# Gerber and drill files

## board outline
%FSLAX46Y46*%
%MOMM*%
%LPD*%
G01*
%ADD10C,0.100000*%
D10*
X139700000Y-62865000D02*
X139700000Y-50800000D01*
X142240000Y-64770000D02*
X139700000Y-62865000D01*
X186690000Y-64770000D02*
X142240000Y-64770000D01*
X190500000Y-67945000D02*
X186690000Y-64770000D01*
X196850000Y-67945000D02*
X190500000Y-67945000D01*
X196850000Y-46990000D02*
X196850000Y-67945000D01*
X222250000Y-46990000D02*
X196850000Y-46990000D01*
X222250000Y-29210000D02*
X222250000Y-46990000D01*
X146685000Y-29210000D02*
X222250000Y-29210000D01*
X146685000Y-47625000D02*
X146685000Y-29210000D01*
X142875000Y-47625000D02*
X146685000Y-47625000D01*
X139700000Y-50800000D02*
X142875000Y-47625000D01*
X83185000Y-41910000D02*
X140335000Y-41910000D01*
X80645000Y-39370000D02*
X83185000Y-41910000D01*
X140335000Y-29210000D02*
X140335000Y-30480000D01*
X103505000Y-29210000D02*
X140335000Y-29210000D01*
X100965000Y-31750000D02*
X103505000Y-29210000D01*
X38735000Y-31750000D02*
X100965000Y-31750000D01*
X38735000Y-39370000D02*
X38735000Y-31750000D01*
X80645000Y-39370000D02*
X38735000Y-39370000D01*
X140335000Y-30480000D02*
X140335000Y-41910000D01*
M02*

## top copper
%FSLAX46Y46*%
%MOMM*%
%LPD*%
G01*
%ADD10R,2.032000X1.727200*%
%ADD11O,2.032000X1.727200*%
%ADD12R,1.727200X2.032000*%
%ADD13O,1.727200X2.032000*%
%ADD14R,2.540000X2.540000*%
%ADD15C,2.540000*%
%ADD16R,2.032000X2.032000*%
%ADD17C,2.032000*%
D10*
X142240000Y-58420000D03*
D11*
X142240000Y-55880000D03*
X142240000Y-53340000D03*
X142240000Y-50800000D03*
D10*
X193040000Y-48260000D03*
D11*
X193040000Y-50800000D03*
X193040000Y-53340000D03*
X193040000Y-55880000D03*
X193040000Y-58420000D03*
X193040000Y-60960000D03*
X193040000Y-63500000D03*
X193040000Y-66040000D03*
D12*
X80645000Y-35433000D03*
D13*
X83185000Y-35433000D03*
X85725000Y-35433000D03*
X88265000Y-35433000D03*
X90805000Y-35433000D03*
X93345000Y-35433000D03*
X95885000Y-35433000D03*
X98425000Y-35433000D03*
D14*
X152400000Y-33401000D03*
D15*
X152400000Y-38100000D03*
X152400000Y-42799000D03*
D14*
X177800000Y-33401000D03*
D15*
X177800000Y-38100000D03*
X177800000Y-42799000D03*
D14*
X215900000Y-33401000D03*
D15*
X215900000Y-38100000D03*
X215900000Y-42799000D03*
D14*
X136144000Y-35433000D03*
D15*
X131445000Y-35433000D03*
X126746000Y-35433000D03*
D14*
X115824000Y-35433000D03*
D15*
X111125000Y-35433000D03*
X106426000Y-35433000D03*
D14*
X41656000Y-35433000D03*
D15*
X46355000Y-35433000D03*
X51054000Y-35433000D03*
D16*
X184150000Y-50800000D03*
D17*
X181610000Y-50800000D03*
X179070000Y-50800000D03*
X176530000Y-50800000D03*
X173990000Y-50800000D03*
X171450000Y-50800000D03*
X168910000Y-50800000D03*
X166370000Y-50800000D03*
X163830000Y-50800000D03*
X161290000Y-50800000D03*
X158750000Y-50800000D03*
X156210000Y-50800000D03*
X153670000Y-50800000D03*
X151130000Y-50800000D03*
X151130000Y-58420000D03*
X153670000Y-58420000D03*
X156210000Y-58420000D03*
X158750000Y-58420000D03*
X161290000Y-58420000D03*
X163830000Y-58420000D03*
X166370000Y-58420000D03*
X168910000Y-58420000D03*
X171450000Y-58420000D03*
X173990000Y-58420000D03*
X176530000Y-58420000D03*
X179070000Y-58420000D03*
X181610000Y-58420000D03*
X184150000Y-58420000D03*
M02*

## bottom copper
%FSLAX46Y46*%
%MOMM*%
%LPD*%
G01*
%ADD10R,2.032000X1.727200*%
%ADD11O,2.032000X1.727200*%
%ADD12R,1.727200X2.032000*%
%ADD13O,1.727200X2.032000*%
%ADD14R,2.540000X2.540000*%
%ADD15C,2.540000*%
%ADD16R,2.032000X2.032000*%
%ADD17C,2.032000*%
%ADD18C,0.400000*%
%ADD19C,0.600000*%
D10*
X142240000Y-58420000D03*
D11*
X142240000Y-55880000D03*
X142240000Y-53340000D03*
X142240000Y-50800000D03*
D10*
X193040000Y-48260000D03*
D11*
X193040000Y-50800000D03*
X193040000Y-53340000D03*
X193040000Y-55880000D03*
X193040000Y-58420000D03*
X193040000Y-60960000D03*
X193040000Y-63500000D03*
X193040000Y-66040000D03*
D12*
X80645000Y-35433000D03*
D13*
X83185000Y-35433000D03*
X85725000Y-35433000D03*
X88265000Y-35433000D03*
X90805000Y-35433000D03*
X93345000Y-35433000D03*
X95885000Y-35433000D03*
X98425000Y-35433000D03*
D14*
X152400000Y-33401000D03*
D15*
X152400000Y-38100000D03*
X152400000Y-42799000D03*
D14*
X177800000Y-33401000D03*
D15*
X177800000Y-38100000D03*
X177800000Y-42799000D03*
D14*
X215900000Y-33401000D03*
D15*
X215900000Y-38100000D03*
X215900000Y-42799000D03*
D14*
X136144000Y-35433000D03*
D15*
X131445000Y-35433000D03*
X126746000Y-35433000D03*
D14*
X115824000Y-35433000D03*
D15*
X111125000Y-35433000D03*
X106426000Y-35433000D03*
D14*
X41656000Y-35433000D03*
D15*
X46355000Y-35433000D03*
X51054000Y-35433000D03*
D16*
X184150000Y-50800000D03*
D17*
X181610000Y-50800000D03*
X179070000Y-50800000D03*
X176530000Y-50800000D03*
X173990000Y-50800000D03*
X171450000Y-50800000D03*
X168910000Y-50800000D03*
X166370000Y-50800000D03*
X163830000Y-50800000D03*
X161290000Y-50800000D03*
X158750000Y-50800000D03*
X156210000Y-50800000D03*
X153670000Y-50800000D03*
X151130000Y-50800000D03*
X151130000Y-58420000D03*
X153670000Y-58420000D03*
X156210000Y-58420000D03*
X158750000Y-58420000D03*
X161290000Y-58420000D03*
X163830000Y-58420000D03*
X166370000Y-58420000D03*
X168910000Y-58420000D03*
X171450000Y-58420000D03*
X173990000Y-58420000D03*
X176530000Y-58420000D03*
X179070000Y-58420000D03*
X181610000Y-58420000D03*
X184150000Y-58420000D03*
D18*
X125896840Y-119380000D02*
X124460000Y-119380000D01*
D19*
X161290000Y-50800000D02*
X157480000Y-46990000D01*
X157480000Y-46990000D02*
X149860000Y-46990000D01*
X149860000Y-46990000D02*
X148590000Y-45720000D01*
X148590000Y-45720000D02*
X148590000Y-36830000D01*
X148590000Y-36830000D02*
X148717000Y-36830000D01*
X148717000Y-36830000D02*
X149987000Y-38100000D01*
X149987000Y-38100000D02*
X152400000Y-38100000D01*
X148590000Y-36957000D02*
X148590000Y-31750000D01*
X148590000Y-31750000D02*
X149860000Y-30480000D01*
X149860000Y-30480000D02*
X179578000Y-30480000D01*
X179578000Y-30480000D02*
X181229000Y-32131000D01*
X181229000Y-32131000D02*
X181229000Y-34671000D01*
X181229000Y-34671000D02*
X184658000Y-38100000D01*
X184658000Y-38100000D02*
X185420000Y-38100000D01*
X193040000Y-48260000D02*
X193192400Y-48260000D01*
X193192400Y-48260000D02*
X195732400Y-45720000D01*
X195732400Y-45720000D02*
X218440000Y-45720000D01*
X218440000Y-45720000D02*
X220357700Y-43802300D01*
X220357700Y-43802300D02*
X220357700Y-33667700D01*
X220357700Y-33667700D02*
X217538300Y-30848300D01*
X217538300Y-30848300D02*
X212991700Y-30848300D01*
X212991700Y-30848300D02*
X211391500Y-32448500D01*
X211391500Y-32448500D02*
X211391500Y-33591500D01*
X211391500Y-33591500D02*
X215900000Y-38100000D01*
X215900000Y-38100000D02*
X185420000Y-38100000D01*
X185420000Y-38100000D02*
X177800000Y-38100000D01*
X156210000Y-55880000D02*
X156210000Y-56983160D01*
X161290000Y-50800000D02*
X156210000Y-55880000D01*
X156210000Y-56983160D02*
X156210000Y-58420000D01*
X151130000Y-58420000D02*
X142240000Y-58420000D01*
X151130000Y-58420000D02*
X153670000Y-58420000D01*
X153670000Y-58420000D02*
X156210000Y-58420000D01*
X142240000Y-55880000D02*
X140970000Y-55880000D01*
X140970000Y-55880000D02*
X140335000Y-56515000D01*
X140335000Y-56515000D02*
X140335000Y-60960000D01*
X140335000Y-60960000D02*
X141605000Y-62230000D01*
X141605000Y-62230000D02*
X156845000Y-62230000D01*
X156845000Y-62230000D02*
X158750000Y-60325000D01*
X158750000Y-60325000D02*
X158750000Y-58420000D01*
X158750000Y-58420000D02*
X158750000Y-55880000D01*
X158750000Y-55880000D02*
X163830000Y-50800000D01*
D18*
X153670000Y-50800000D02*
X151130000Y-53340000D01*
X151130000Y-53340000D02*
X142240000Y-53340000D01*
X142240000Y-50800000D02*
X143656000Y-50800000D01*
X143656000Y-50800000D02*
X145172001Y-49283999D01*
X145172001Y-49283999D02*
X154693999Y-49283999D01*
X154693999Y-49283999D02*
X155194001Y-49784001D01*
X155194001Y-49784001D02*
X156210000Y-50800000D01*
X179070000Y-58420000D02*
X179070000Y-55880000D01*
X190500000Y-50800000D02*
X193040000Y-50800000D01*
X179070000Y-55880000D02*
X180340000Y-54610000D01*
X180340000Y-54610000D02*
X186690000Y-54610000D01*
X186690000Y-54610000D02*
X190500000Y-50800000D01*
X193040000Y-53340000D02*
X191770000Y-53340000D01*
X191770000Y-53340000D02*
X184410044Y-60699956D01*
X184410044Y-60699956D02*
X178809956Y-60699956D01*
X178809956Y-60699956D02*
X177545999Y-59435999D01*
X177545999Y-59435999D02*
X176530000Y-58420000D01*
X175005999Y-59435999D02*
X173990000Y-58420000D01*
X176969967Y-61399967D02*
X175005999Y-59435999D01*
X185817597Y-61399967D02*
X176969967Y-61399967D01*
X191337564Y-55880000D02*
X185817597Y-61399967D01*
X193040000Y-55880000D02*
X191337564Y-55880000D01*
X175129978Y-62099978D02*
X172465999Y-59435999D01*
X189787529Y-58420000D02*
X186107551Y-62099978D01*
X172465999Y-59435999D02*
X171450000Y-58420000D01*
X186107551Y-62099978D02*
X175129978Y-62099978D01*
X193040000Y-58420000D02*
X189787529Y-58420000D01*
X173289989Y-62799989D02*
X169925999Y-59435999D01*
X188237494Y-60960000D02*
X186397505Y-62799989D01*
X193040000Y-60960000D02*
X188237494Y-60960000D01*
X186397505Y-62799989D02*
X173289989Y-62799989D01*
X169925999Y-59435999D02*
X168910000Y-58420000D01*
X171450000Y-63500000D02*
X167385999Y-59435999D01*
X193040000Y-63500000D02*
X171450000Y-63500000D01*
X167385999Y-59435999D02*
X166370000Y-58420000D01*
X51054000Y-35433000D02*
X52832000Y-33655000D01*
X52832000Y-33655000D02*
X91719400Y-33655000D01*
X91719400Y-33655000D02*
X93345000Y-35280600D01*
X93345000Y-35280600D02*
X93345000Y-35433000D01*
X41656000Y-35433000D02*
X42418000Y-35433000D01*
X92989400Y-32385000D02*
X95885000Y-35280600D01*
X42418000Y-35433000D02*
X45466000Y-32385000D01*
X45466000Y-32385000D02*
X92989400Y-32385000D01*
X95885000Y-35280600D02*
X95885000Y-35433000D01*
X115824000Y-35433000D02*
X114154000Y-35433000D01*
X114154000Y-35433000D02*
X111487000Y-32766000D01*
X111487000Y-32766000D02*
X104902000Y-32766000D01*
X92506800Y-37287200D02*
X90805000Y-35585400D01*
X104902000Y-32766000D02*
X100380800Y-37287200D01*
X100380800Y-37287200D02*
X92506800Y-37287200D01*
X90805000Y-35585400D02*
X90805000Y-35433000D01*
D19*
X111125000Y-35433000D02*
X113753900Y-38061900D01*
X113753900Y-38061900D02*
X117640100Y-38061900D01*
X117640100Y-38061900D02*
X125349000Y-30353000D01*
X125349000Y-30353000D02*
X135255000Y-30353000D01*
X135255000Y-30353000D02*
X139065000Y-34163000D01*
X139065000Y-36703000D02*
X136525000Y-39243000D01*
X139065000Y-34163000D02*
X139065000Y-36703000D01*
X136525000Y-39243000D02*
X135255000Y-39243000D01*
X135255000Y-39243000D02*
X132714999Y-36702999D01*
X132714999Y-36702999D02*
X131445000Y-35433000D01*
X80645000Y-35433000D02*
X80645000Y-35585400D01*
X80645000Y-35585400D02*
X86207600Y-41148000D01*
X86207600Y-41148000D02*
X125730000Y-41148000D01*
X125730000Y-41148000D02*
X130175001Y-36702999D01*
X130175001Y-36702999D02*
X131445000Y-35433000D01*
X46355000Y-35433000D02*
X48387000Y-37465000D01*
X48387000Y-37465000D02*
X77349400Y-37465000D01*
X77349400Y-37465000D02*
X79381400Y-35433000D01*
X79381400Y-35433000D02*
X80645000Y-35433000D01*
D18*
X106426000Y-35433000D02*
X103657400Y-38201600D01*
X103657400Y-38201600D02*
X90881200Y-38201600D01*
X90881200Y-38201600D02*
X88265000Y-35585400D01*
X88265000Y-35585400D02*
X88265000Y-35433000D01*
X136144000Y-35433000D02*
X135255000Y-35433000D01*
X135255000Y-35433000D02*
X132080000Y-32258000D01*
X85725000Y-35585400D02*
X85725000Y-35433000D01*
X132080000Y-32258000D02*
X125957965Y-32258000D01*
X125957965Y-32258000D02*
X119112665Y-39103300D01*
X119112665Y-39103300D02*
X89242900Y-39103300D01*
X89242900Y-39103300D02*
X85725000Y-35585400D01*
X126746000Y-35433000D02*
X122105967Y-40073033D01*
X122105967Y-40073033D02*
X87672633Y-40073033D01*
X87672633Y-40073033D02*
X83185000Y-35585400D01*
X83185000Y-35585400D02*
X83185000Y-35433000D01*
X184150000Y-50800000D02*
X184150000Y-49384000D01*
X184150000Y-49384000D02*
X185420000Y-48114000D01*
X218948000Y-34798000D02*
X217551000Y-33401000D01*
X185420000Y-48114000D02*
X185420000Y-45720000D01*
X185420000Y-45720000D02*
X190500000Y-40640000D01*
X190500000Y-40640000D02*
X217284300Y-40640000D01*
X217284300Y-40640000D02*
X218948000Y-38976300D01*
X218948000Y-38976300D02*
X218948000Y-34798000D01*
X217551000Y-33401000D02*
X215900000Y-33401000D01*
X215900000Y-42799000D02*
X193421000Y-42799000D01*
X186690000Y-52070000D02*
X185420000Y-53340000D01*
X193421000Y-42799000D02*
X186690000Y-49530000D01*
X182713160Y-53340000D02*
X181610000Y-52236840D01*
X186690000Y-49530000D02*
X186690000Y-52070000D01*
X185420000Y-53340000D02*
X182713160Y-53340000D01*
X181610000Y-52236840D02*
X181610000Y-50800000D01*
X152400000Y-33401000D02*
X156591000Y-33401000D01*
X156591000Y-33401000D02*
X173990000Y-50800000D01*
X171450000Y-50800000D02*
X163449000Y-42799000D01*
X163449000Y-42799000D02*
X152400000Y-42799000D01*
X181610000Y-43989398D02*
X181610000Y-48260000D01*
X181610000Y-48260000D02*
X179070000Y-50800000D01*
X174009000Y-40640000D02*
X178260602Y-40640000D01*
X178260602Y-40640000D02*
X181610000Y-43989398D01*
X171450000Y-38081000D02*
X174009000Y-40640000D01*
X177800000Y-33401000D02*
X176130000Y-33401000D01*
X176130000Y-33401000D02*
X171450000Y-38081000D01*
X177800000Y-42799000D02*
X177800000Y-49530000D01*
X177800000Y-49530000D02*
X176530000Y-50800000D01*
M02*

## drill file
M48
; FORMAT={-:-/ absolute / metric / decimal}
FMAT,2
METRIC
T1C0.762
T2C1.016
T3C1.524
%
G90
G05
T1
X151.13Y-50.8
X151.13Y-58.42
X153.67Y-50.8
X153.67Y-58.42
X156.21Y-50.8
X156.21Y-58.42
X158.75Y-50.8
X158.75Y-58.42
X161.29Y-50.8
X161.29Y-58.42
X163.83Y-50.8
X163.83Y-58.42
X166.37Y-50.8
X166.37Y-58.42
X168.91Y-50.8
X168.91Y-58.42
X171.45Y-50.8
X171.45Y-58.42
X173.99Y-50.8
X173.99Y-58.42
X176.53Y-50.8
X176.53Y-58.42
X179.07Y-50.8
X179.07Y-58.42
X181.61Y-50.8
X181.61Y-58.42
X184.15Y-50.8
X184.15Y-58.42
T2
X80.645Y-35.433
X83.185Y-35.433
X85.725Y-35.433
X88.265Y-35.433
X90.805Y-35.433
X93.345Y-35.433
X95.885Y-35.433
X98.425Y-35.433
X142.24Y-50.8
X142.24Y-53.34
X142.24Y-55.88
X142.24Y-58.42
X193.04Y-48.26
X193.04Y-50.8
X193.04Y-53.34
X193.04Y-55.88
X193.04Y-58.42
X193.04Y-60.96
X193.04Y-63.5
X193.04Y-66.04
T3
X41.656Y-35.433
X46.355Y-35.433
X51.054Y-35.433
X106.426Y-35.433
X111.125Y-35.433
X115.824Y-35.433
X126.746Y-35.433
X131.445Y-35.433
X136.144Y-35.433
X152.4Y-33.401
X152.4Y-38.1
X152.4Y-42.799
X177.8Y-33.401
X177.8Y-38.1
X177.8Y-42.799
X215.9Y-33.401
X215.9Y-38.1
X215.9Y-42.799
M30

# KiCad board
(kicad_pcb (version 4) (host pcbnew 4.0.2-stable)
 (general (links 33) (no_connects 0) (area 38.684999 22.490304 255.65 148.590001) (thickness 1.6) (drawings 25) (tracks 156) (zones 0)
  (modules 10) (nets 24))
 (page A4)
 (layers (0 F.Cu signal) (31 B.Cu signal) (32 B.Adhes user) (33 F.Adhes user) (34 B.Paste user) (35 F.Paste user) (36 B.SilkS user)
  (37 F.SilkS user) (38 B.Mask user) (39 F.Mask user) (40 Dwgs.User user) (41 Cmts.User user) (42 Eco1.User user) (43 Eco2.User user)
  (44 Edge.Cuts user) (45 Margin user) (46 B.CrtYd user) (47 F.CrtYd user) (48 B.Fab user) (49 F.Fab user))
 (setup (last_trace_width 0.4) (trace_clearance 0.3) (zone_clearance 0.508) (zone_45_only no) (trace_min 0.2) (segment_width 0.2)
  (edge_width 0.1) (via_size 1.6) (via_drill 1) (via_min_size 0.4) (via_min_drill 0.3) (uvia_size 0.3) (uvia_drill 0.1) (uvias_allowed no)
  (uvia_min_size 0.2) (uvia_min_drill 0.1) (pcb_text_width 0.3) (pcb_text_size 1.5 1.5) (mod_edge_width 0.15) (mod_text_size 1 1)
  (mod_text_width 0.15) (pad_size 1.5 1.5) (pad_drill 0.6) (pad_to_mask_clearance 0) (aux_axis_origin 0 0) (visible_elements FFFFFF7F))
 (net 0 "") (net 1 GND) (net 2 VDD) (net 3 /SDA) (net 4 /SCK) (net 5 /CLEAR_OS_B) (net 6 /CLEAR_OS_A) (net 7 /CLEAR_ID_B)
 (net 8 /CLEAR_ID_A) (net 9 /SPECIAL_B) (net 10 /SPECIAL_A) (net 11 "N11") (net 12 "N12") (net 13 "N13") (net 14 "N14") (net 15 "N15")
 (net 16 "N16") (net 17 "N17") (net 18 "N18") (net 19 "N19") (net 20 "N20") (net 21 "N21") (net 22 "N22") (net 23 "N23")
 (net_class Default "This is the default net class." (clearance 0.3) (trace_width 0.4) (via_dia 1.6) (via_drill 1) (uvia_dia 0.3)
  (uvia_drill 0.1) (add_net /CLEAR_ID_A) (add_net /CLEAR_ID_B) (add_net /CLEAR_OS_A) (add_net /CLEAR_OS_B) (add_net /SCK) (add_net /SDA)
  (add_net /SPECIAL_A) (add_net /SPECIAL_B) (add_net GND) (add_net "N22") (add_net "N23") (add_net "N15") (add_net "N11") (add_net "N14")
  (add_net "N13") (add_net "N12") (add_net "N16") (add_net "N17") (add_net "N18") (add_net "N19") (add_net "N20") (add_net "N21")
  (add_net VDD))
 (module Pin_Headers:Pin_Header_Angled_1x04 (layer F.Cu) (at 142.24 58.42 180)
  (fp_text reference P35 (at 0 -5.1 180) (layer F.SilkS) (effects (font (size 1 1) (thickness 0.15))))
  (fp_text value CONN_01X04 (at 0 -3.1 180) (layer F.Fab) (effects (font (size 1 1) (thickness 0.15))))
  (pad 1 thru_hole rect (at 0 0 180) (size 2.032 1.7272) (drill 1.016) (layers *.Cu *.Mask F.SilkS) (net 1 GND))
  (pad 2 thru_hole oval (at 0 2.54 180) (size 2.032 1.7272) (drill 1.016) (layers *.Cu *.Mask F.SilkS) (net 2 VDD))
  (pad 3 thru_hole oval (at 0 5.08 180) (size 2.032 1.7272) (drill 1.016) (layers *.Cu *.Mask F.SilkS) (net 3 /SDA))
  (pad 4 thru_hole oval (at 0 7.62 180) (size 2.032 1.7272) (drill 1.016) (layers *.Cu *.Mask F.SilkS) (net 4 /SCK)))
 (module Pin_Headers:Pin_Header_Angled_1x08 (layer F.Cu) (at 193.04 48.26)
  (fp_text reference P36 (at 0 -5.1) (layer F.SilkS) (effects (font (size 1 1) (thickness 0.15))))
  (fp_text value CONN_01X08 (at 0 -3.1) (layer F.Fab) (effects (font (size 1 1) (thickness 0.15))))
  (pad 1 thru_hole rect (at 0 0) (size 2.032 1.7272) (drill 1.016) (layers *.Cu *.Mask F.SilkS) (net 1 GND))
  (pad 2 thru_hole oval (at 0 2.54) (size 2.032 1.7272) (drill 1.016) (layers *.Cu *.Mask F.SilkS) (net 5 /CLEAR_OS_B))
  (pad 3 thru_hole oval (at 0 5.08) (size 2.032 1.7272) (drill 1.016) (layers *.Cu *.Mask F.SilkS) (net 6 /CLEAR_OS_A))
  (pad 4 thru_hole oval (at 0 7.62) (size 2.032 1.7272) (drill 1.016) (layers *.Cu *.Mask F.SilkS) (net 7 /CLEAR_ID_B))
  (pad 5 thru_hole oval (at 0 10.16) (size 2.032 1.7272) (drill 1.016) (layers *.Cu *.Mask F.SilkS) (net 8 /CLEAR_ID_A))
  (pad 6 thru_hole oval (at 0 12.7) (size 2.032 1.7272) (drill 1.016) (layers *.Cu *.Mask F.SilkS) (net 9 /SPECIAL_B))
  (pad 7 thru_hole oval (at 0 15.24) (size 2.032 1.7272) (drill 1.016) (layers *.Cu *.Mask F.SilkS) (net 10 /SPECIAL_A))
  (pad 8 thru_hole oval (at 0 17.78) (size 2.032 1.7272) (drill 1.016) (layers *.Cu *.Mask F.SilkS)))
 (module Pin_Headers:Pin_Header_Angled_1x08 (layer F.Cu) (at 80.645 35.433 90)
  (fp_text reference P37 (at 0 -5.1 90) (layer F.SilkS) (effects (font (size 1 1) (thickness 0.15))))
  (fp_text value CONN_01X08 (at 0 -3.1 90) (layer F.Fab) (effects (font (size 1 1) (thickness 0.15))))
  (pad 1 thru_hole rect (at 0 0 90) (size 2.032 1.7272) (drill 1.016) (layers *.Cu *.Mask F.SilkS) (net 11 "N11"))
  (pad 2 thru_hole oval (at 0 2.54 90) (size 2.032 1.7272) (drill 1.016) (layers *.Cu *.Mask F.SilkS) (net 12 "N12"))
  (pad 3 thru_hole oval (at 0 5.08 90) (size 2.032 1.7272) (drill 1.016) (layers *.Cu *.Mask F.SilkS) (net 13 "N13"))
  (pad 4 thru_hole oval (at 0 7.62 90) (size 2.032 1.7272) (drill 1.016) (layers *.Cu *.Mask F.SilkS) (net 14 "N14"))
  (pad 5 thru_hole oval (at 0 10.16 90) (size 2.032 1.7272) (drill 1.016) (layers *.Cu *.Mask F.SilkS) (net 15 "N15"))
  (pad 6 thru_hole oval (at 0 12.7 90) (size 2.032 1.7272) (drill 1.016) (layers *.Cu *.Mask F.SilkS) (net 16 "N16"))
  (pad 7 thru_hole oval (at 0 15.24 90) (size 2.032 1.7272) (drill 1.016) (layers *.Cu *.Mask F.SilkS) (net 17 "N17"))
  (pad 8 thru_hole oval (at 0 17.78 90) (size 2.032 1.7272) (drill 1.016) (layers *.Cu *.Mask F.SilkS)))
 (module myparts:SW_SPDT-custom (layer F.Cu) (at 152.4 38.1 270)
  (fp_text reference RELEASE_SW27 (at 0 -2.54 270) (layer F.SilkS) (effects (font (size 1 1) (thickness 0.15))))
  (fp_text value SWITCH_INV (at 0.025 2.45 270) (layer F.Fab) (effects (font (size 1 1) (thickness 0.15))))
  (pad 1 thru_hole rect (at -4.699 0 270) (size 2.54 2.54) (drill 1.524) (layers *.Cu *.Mask F.SilkS) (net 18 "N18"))
  (pad 2 thru_hole circle (at 0 0 270) (size 2.54 2.54) (drill 1.524) (layers *.Cu *.Mask F.SilkS) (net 1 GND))
  (pad 3 thru_hole circle (at 4.699 0 270) (size 2.54 2.54) (drill 1.524) (layers *.Cu *.Mask F.SilkS) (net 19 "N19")))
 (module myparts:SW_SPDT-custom (layer F.Cu) (at 177.8 38.1 270)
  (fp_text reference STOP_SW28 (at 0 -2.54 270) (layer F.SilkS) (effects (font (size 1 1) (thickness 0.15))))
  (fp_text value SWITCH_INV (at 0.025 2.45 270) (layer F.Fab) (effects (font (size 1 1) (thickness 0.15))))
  (pad 1 thru_hole rect (at -4.699 0 270) (size 2.54 2.54) (drill 1.524) (layers *.Cu *.Mask F.SilkS) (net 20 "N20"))
  (pad 2 thru_hole circle (at 0 0 270) (size 2.54 2.54) (drill 1.524) (layers *.Cu *.Mask F.SilkS) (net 1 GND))
  (pad 3 thru_hole circle (at 4.699 0 270) (size 2.54 2.54) (drill 1.524) (layers *.Cu *.Mask F.SilkS) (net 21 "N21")))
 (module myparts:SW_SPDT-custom (layer F.Cu) (at 215.9 38.1 270)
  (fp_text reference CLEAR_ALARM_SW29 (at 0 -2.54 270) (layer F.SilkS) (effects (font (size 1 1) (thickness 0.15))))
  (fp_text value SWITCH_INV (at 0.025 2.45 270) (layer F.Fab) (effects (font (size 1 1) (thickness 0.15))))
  (pad 1 thru_hole rect (at -4.699 0 270) (size 2.54 2.54) (drill 1.524) (layers *.Cu *.Mask F.SilkS) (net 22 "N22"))
  (pad 2 thru_hole circle (at 0 0 270) (size 2.54 2.54) (drill 1.524) (layers *.Cu *.Mask F.SilkS) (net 1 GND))
  (pad 3 thru_hole circle (at 4.699 0 270) (size 2.54 2.54) (drill 1.524) (layers *.Cu *.Mask F.SilkS) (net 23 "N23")))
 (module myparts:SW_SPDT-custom (layer F.Cu) (at 131.445 35.433 180)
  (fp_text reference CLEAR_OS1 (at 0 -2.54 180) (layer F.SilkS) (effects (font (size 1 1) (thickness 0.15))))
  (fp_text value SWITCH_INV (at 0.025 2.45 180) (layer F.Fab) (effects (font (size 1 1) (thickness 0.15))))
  (pad 1 thru_hole rect (at -4.699 0 180) (size 2.54 2.54) (drill 1.524) (layers *.Cu *.Mask F.SilkS) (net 13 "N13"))
  (pad 2 thru_hole circle (at 0 0 180) (size 2.54 2.54) (drill 1.524) (layers *.Cu *.Mask F.SilkS) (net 11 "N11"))
  (pad 3 thru_hole circle (at 4.699 0 180) (size 2.54 2.54) (drill 1.524) (layers *.Cu *.Mask F.SilkS) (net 12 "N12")))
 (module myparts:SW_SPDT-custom (layer F.Cu) (at 111.125 35.433 180)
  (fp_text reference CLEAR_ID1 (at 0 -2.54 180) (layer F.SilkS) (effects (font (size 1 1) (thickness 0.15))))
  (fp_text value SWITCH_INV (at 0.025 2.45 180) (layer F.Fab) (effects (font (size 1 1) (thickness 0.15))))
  (pad 1 thru_hole rect (at -4.699 0 180) (size 2.54 2.54) (drill 1.524) (layers *.Cu *.Mask F.SilkS) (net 15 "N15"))
  (pad 2 thru_hole circle (at 0 0 180) (size 2.54 2.54) (drill 1.524) (layers *.Cu *.Mask F.SilkS) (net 11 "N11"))
  (pad 3 thru_hole circle (at 4.699 0 180) (size 2.54 2.54) (drill 1.524) (layers *.Cu *.Mask F.SilkS) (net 14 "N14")))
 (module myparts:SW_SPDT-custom (layer F.Cu) (at 46.355 35.433)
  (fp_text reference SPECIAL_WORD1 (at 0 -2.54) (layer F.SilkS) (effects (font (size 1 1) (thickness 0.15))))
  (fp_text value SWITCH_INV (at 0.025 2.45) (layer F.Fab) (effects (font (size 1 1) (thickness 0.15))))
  (pad 1 thru_hole rect (at -4.699 0) (size 2.54 2.54) (drill 1.524) (layers *.Cu *.Mask F.SilkS) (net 17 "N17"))
  (pad 2 thru_hole circle (at 0 0) (size 2.54 2.54) (drill 1.524) (layers *.Cu *.Mask F.SilkS) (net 11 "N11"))
  (pad 3 thru_hole circle (at 4.699 0) (size 2.54 2.54) (drill 1.524) (layers *.Cu *.Mask F.SilkS) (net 16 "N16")))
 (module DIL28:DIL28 (layer F.Cu) (at 184.15 50.8 180)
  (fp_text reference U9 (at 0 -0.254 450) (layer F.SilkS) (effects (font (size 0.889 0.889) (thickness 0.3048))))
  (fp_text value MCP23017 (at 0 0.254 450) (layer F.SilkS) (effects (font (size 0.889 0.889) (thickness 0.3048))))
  (pad 1 thru_hole rect (at 0 0 180) (size 2.032 2.032) (drill 0.762) (layers *.Cu *.Mask F.SilkS) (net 22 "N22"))
  (pad 2 thru_hole circle (at 2.54 0 180) (size 2.032 2.032) (drill 0.762) (layers *.Cu *.Mask F.SilkS) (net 23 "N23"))
  (pad 3 thru_hole circle (at 5.08 0 180) (size 2.032 2.032) (drill 0.762) (layers *.Cu *.Mask F.SilkS) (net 20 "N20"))
  (pad 4 thru_hole circle (at 7.62 0 180) (size 2.032 2.032) (drill 0.762) (layers *.Cu *.Mask F.SilkS) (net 21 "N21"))
  (pad 5 thru_hole circle (at 10.16 0 180) (size 2.032 2.032) (drill 0.762) (layers *.Cu *.Mask F.SilkS) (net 18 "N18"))
  (pad 6 thru_hole circle (at 12.7 0 180) (size 2.032 2.032) (drill 0.762) (layers *.Cu *.Mask F.SilkS) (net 19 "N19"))
  (pad 7 thru_hole circle (at 15.24 0 180) (size 2.032 2.032) (drill 0.762) (layers *.Cu *.Mask F.SilkS))
  (pad 8 thru_hole circle (at 17.78 0 180) (size 2.032 2.032) (drill 0.762) (layers *.Cu *.Mask F.SilkS))
  (pad 9 thru_hole circle (at 20.32 0 180) (size 2.032 2.032) (drill 0.762) (layers *.Cu *.Mask F.SilkS) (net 2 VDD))
  (pad 10 thru_hole circle (at 22.86 0 180) (size 2.032 2.032) (drill 0.762) (layers *.Cu *.Mask F.SilkS) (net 1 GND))
  (pad 11 thru_hole circle (at 25.4 0 180) (size 2.032 2.032) (drill 0.762) (layers *.Cu *.Mask F.SilkS))
  (pad 12 thru_hole circle (at 27.94 0 180) (size 2.032 2.032) (drill 0.762) (layers *.Cu *.Mask F.SilkS) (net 4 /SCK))
  (pad 13 thru_hole circle (at 30.48 0 180) (size 2.032 2.032) (drill 0.762) (layers *.Cu *.Mask F.SilkS) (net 3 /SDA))
  (pad 14 thru_hole circle (at 33.02 0 180) (size 2.032 2.032) (drill 0.762) (layers *.Cu *.Mask F.SilkS))
  (pad 15 thru_hole circle (at 33.02 -7.62) (size 2.032 2.032) (drill 0.762) (layers *.Cu *.Mask F.SilkS) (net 1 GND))
  (pad 16 thru_hole circle (at 30.48 -7.62) (size 2.032 2.032) (drill 0.762) (layers *.Cu *.Mask F.SilkS) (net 1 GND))
  (pad 17 thru_hole circle (at 27.94 -7.62) (size 2.032 2.032) (drill 0.762) (layers *.Cu *.Mask F.SilkS) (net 1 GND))
  (pad 18 thru_hole circle (at 25.4 -7.62) (size 2.032 2.032) (drill 0.762) (layers *.Cu *.Mask F.SilkS) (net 2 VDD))
  (pad 19 thru_hole circle (at 22.86 -7.62) (size 2.032 2.032) (drill 0.762) (layers *.Cu *.Mask F.SilkS))
  (pad 20 thru_hole circle (at 20.32 -7.62) (size 2.032 2.032) (drill 0.762) (layers *.Cu *.Mask F.SilkS))
  (pad 21 thru_hole circle (at 17.78 -7.62) (size 2.032 2.032) (drill 0.762) (layers *.Cu *.Mask F.SilkS) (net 10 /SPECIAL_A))
  (pad 22 thru_hole circle (at 15.24 -7.62) (size 2.032 2.032) (drill 0.762) (layers *.Cu *.Mask F.SilkS) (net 9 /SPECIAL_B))
  (pad 23 thru_hole circle (at 12.7 -7.62) (size 2.032 2.032) (drill 0.762) (layers *.Cu *.Mask F.SilkS) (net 8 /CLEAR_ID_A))
  (pad 24 thru_hole circle (at 10.16 -7.62) (size 2.032 2.032) (drill 0.762) (layers *.Cu *.Mask F.SilkS) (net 7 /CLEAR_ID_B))
  (pad 25 thru_hole circle (at 7.62 -7.62) (size 2.032 2.032) (drill 0.762) (layers *.Cu *.Mask F.SilkS) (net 6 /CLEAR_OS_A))
  (pad 26 thru_hole circle (at 5.08 -7.62) (size 2.032 2.032) (drill 0.762) (layers *.Cu *.Mask F.SilkS) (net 5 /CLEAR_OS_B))
  (pad 27 thru_hole circle (at 2.54 -7.62) (size 2.032 2.032) (drill 0.762) (layers *.Cu *.Mask F.SilkS))
  (pad 28 thru_hole circle (at 0 -7.62) (size 2.032 2.032) (drill 0.762) (layers *.Cu *.Mask F.SilkS)))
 (gr_line (start 139.7 62.865) (end 139.7 50.8) (layer Edge.Cuts) (width 0.1))
 (gr_line (start 142.24 64.77) (end 139.7 62.865) (layer Edge.Cuts) (width 0.1))
 (gr_line (start 186.69 64.77) (end 142.24 64.77) (layer Edge.Cuts) (width 0.1))
 (gr_line (start 190.5 67.945) (end 186.69 64.77) (layer Edge.Cuts) (width 0.1))
 (gr_line (start 196.85 67.945) (end 190.5 67.945) (layer Edge.Cuts) (width 0.1))
 (gr_line (start 196.85 46.99) (end 196.85 67.945) (layer Edge.Cuts) (width 0.1))
 (gr_line (start 222.25 46.99) (end 196.85 46.99) (layer Edge.Cuts) (width 0.1))
 (gr_line (start 222.25 29.21) (end 222.25 46.99) (layer Edge.Cuts) (width 0.1))
 (gr_line (start 146.685 29.21) (end 222.25 29.21) (layer Edge.Cuts) (width 0.1))
 (gr_line (start 146.685 47.625) (end 146.685 29.21) (layer Edge.Cuts) (width 0.1))
 (gr_line (start 142.875 47.625) (end 146.685 47.625) (layer Edge.Cuts) (width 0.1))
 (gr_line (start 139.7 50.8) (end 142.875 47.625) (layer Edge.Cuts) (width 0.1))
 (gr_line (start 83.185 41.91) (end 140.335 41.91) (layer Edge.Cuts) (width 0.1))
 (gr_line (start 80.645 39.37) (end 83.185 41.91) (layer Edge.Cuts) (width 0.1))
 (gr_line (start 140.335 29.21) (end 140.335 30.48) (layer Edge.Cuts) (width 0.1))
 (gr_line (start 103.505 29.21) (end 140.335 29.21) (layer Edge.Cuts) (width 0.1))
 (gr_line (start 100.965 31.75) (end 103.505 29.21) (layer Edge.Cuts) (width 0.1))
 (gr_line (start 38.735 31.75) (end 100.965 31.75) (layer Edge.Cuts) (width 0.1))
 (gr_line (start 38.735 39.37) (end 38.735 31.75) (layer Edge.Cuts) (width 0.1))
 (gr_line (start 80.645 39.37) (end 38.735 39.37) (layer Edge.Cuts) (width 0.1))
 (gr_line (start 140.335 30.48) (end 140.335 41.91) (layer Edge.Cuts) (width 0.1))
 (segment (start 125.89684 119.38) (end 124.46 119.38) (width 0.4) (layer B.Cu) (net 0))
 (segment (start 161.29 50.8) (end 157.48 46.99) (width 0.6) (layer B.Cu) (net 1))
 (segment (start 157.48 46.99) (end 149.86 46.99) (width 0.6) (layer B.Cu) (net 1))
 (segment (start 149.86 46.99) (end 148.59 45.72) (width 0.6) (layer B.Cu) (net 1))
 (segment (start 148.59 45.72) (end 148.59 36.83) (width 0.6) (layer B.Cu) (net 1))
 (segment (start 148.59 36.83) (end 148.717 36.83) (width 0.6) (layer B.Cu) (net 1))
 (segment (start 148.717 36.83) (end 149.987 38.1) (width 0.6) (layer B.Cu) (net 1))
 (segment (start 149.987 38.1) (end 152.4 38.1) (width 0.6) (layer B.Cu) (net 1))
 (segment (start 148.59 36.957) (end 148.59 31.75) (width 0.6) (layer B.Cu) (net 1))
 (segment (start 148.59 31.75) (end 149.86 30.48) (width 0.6) (layer B.Cu) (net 1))
 (segment (start 149.86 30.48) (end 179.578 30.48) (width 0.6) (layer B.Cu) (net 1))
 (segment (start 179.578 30.48) (end 181.229 32.131) (width 0.6) (layer B.Cu) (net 1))
 (segment (start 181.229 32.131) (end 181.229 34.671) (width 0.6) (layer B.Cu) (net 1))
 (segment (start 181.229 34.671) (end 184.658 38.1) (width 0.6) (layer B.Cu) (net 1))
 (segment (start 184.658 38.1) (end 185.42 38.1) (width 0.6) (layer B.Cu) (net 1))
 (segment (start 193.04 48.26) (end 193.1924 48.26) (width 0.6) (layer B.Cu) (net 1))
 (segment (start 193.1924 48.26) (end 195.7324 45.72) (width 0.6) (layer B.Cu) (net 1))
 (segment (start 195.7324 45.72) (end 218.44 45.72) (width 0.6) (layer B.Cu) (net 1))
 (segment (start 218.44 45.72) (end 220.3577 43.8023) (width 0.6) (layer B.Cu) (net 1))
 (segment (start 220.3577 43.8023) (end 220.3577 33.6677) (width 0.6) (layer B.Cu) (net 1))
 (segment (start 220.3577 33.6677) (end 217.5383 30.8483) (width 0.6) (layer B.Cu) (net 1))
 (segment (start 217.5383 30.8483) (end 212.9917 30.8483) (width 0.6) (layer B.Cu) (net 1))
 (segment (start 212.9917 30.8483) (end 211.3915 32.4485) (width 0.6) (layer B.Cu) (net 1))
 (segment (start 211.3915 32.4485) (end 211.3915 33.5915) (width 0.6) (layer B.Cu) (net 1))
 (segment (start 211.3915 33.5915) (end 215.9 38.1) (width 0.6) (layer B.Cu) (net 1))
 (segment (start 215.9 38.1) (end 185.42 38.1) (width 0.6) (layer B.Cu) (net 1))
 (segment (start 185.42 38.1) (end 177.8 38.1) (width 0.6) (layer B.Cu) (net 1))
 (segment (start 156.21 55.88) (end 156.21 56.98316) (width 0.6) (layer B.Cu) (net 1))
 (segment (start 161.29 50.8) (end 156.21 55.88) (width 0.6) (layer B.Cu) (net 1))
 (segment (start 156.21 56.98316) (end 156.21 58.42) (width 0.6) (layer B.Cu) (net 1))
 (segment (start 151.13 58.42) (end 142.24 58.42) (width 0.6) (layer B.Cu) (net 1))
 (segment (start 151.13 58.42) (end 153.67 58.42) (width 0.6) (layer B.Cu) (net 1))
 (segment (start 153.67 58.42) (end 156.21 58.42) (width 0.6) (layer B.Cu) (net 1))
 (segment (start 142.24 55.88) (end 140.97 55.88) (width 0.6) (layer B.Cu) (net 2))
 (segment (start 140.97 55.88) (end 140.335 56.515) (width 0.6) (layer B.Cu) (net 2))
 (segment (start 140.335 56.515) (end 140.335 60.96) (width 0.6) (layer B.Cu) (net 2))
 (segment (start 140.335 60.96) (end 141.605 62.23) (width 0.6) (layer B.Cu) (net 2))
 (segment (start 141.605 62.23) (end 156.845 62.23) (width 0.6) (layer B.Cu) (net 2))
 (segment (start 156.845 62.23) (end 158.75 60.325) (width 0.6) (layer B.Cu) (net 2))
 (segment (start 158.75 60.325) (end 158.75 58.42) (width 0.6) (layer B.Cu) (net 2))
 (segment (start 158.75 58.42) (end 158.75 55.88) (width 0.6) (layer B.Cu) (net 2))
 (segment (start 158.75 55.88) (end 163.83 50.8) (width 0.6) (layer B.Cu) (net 2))
 (segment (start 153.67 50.8) (end 151.13 53.34) (width 0.4) (layer B.Cu) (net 3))
 (segment (start 151.13 53.34) (end 142.24 53.34) (width 0.4) (layer B.Cu) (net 3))
 (segment (start 142.24 50.8) (end 143.656 50.8) (width 0.4) (layer B.Cu) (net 4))
 (segment (start 143.656 50.8) (end 145.172001 49.283999) (width 0.4) (layer B.Cu) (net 4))
 (segment (start 145.172001 49.283999) (end 154.693999 49.283999) (width 0.4) (layer B.Cu) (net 4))
 (segment (start 154.693999 49.283999) (end 155.194001 49.784001) (width 0.4) (layer B.Cu) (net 4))
 (segment (start 155.194001 49.784001) (end 156.21 50.8) (width 0.4) (layer B.Cu) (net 4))
 (segment (start 179.07 58.42) (end 179.07 55.88) (width 0.4) (layer B.Cu) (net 5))
 (segment (start 190.5 50.8) (end 193.04 50.8) (width 0.4) (layer B.Cu) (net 5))
 (segment (start 179.07 55.88) (end 180.34 54.61) (width 0.4) (layer B.Cu) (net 5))
 (segment (start 180.34 54.61) (end 186.69 54.61) (width 0.4) (layer B.Cu) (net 5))
 (segment (start 186.69 54.61) (end 190.5 50.8) (width 0.4) (layer B.Cu) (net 5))
 (segment (start 193.04 53.34) (end 191.77 53.34) (width 0.4) (layer B.Cu) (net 6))
 (segment (start 191.77 53.34) (end 184.410044 60.699956) (width 0.4) (layer B.Cu) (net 6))
 (segment (start 184.410044 60.699956) (end 178.809956 60.699956) (width 0.4) (layer B.Cu) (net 6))
 (segment (start 178.809956 60.699956) (end 177.545999 59.435999) (width 0.4) (layer B.Cu) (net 6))
 (segment (start 177.545999 59.435999) (end 176.53 58.42) (width 0.4) (layer B.Cu) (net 6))
 (segment (start 175.005999 59.435999) (end 173.99 58.42) (width 0.4) (layer B.Cu) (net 7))
 (segment (start 176.969967 61.399967) (end 175.005999 59.435999) (width 0.4) (layer B.Cu) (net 7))
 (segment (start 185.817597 61.399967) (end 176.969967 61.399967) (width 0.4) (layer B.Cu) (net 7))
 (segment (start 191.337564 55.88) (end 185.817597 61.399967) (width 0.4) (layer B.Cu) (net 7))
 (segment (start 193.04 55.88) (end 191.337564 55.88) (width 0.4) (layer B.Cu) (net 7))
 (segment (start 175.129978 62.099978) (end 172.465999 59.435999) (width 0.4) (layer B.Cu) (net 8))
 (segment (start 189.787529 58.42) (end 186.107551 62.099978) (width 0.4) (layer B.Cu) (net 8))
 (segment (start 172.465999 59.435999) (end 171.45 58.42) (width 0.4) (layer B.Cu) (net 8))
 (segment (start 186.107551 62.099978) (end 175.129978 62.099978) (width 0.4) (layer B.Cu) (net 8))
 (segment (start 193.04 58.42) (end 189.787529 58.42) (width 0.4) (layer B.Cu) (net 8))
 (segment (start 173.289989 62.799989) (end 169.925999 59.435999) (width 0.4) (layer B.Cu) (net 9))
 (segment (start 188.237494 60.96) (end 186.397505 62.799989) (width 0.4) (layer B.Cu) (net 9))
 (segment (start 193.04 60.96) (end 188.237494 60.96) (width 0.4) (layer B.Cu) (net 9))
 (segment (start 186.397505 62.799989) (end 173.289989 62.799989) (width 0.4) (layer B.Cu) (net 9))
 (segment (start 169.925999 59.435999) (end 168.91 58.42) (width 0.4) (layer B.Cu) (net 9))
 (segment (start 171.45 63.5) (end 167.385999 59.435999) (width 0.4) (layer B.Cu) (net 10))
 (segment (start 193.04 63.5) (end 171.45 63.5) (width 0.4) (layer B.Cu) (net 10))
 (segment (start 167.385999 59.435999) (end 166.37 58.42) (width 0.4) (layer B.Cu) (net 10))
 (segment (start 51.054 35.433) (end 52.832 33.655) (width 0.4) (layer B.Cu) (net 16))
 (segment (start 52.832 33.655) (end 91.7194 33.655) (width 0.4) (layer B.Cu) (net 16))
 (segment (start 91.7194 33.655) (end 93.345 35.2806) (width 0.4) (layer B.Cu) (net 16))
 (segment (start 93.345 35.2806) (end 93.345 35.433) (width 0.4) (layer B.Cu) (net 16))
 (segment (start 41.656 35.433) (end 42.418 35.433) (width 0.4) (layer B.Cu) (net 17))
 (segment (start 92.9894 32.385) (end 95.885 35.2806) (width 0.4) (layer B.Cu) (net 17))
 (segment (start 42.418 35.433) (end 45.466 32.385) (width 0.4) (layer B.Cu) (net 17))
 (segment (start 45.466 32.385) (end 92.9894 32.385) (width 0.4) (layer B.Cu) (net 17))
 (segment (start 95.885 35.2806) (end 95.885 35.433) (width 0.4) (layer B.Cu) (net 17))
 (segment (start 115.824 35.433) (end 114.154 35.433) (width 0.4) (layer B.Cu) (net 15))
 (segment (start 114.154 35.433) (end 111.487 32.766) (width 0.4) (layer B.Cu) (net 15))
 (segment (start 111.487 32.766) (end 104.902 32.766) (width 0.4) (layer B.Cu) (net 15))
 (segment (start 92.5068 37.2872) (end 90.805 35.5854) (width 0.4) (layer B.Cu) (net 15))
 (segment (start 104.902 32.766) (end 100.3808 37.2872) (width 0.4) (layer B.Cu) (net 15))
 (segment (start 100.3808 37.2872) (end 92.5068 37.2872) (width 0.4) (layer B.Cu) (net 15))
 (segment (start 90.805 35.5854) (end 90.805 35.433) (width 0.4) (layer B.Cu) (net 15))
 (segment (start 111.125 35.433) (end 113.7539 38.0619) (width 0.6) (layer B.Cu) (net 11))
 (segment (start 113.7539 38.0619) (end 117.6401 38.0619) (width 0.6) (layer B.Cu) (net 11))
 (segment (start 117.6401 38.0619) (end 125.349 30.353) (width 0.6) (layer B.Cu) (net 11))
 (segment (start 125.349 30.353) (end 135.255 30.353) (width 0.6) (layer B.Cu) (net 11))
 (segment (start 135.255 30.353) (end 139.065 34.163) (width 0.6) (layer B.Cu) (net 11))
 (segment (start 139.065 36.703) (end 136.525 39.243) (width 0.6) (layer B.Cu) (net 11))
 (segment (start 139.065 34.163) (end 139.065 36.703) (width 0.6) (layer B.Cu) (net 11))
 (segment (start 136.525 39.243) (end 135.255 39.243) (width 0.6) (layer B.Cu) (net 11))
 (segment (start 135.255 39.243) (end 132.714999 36.702999) (width 0.6) (layer B.Cu) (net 11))
 (segment (start 132.714999 36.702999) (end 131.445 35.433) (width 0.6) (layer B.Cu) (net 11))
 (segment (start 80.645 35.433) (end 80.645 35.5854) (width 0.6) (layer B.Cu) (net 11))
 (segment (start 80.645 35.5854) (end 86.2076 41.148) (width 0.6) (layer B.Cu) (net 11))
 (segment (start 86.2076 41.148) (end 125.73 41.148) (width 0.6) (layer B.Cu) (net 11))
 (segment (start 125.73 41.148) (end 130.175001 36.702999) (width 0.6) (layer B.Cu) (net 11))
 (segment (start 130.175001 36.702999) (end 131.445 35.433) (width 0.6) (layer B.Cu) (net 11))
 (segment (start 46.355 35.433) (end 48.387 37.465) (width 0.6) (layer B.Cu) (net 11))
 (segment (start 48.387 37.465) (end 77.3494 37.465) (width 0.6) (layer B.Cu) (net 11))
 (segment (start 77.3494 37.465) (end 79.3814 35.433) (width 0.6) (layer B.Cu) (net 11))
 (segment (start 79.3814 35.433) (end 80.645 35.433) (width 0.6) (layer B.Cu) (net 11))
 (segment (start 106.426 35.433) (end 103.6574 38.2016) (width 0.4) (layer B.Cu) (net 14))
 (segment (start 103.6574 38.2016) (end 90.8812 38.2016) (width 0.4) (layer B.Cu) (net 14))
 (segment (start 90.8812 38.2016) (end 88.265 35.5854) (width 0.4) (layer B.Cu) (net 14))
 (segment (start 88.265 35.5854) (end 88.265 35.433) (width 0.4) (layer B.Cu) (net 14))
 (segment (start 136.144 35.433) (end 135.255 35.433) (width 0.4) (layer B.Cu) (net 13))
 (segment (start 135.255 35.433) (end 132.08 32.258) (width 0.4) (layer B.Cu) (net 13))
 (segment (start 85.725 35.5854) (end 85.725 35.433) (width 0.4) (layer B.Cu) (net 13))
 (segment (start 132.08 32.258) (end 125.957965 32.258) (width 0.4) (layer B.Cu) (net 13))
 (segment (start 125.957965 32.258) (end 119.112665 39.1033) (width 0.4) (layer B.Cu) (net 13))
 (segment (start 119.112665 39.1033) (end 89.2429 39.1033) (width 0.4) (layer B.Cu) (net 13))
 (segment (start 89.2429 39.1033) (end 85.725 35.5854) (width 0.4) (layer B.Cu) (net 13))
 (segment (start 126.746 35.433) (end 122.105967 40.073033) (width 0.4) (layer B.Cu) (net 12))
 (segment (start 122.105967 40.073033) (end 87.672633 40.073033) (width 0.4) (layer B.Cu) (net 12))
 (segment (start 87.672633 40.073033) (end 83.185 35.5854) (width 0.4) (layer B.Cu) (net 12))
 (segment (start 83.185 35.5854) (end 83.185 35.433) (width 0.4) (layer B.Cu) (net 12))
 (segment (start 184.15 50.8) (end 184.15 49.384) (width 0.4) (layer B.Cu) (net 22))
 (segment (start 184.15 49.384) (end 185.42 48.114) (width 0.4) (layer B.Cu) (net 22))
 (segment (start 218.948 34.798) (end 217.551 33.401) (width 0.4) (layer B.Cu) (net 22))
 (segment (start 185.42 48.114) (end 185.42 45.72) (width 0.4) (layer B.Cu) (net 22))
 (segment (start 185.42 45.72) (end 190.5 40.64) (width 0.4) (layer B.Cu) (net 22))
 (segment (start 190.5 40.64) (end 217.2843 40.64) (width 0.4) (layer B.Cu) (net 22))
 (segment (start 217.2843 40.64) (end 218.948 38.9763) (width 0.4) (layer B.Cu) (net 22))
 (segment (start 218.948 38.9763) (end 218.948 34.798) (width 0.4) (layer B.Cu) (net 22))
 (segment (start 217.551 33.401) (end 215.9 33.401) (width 0.4) (layer B.Cu) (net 22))
 (segment (start 215.9 42.799) (end 193.421 42.799) (width 0.4) (layer B.Cu) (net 23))
 (segment (start 186.69 52.07) (end 185.42 53.34) (width 0.4) (layer B.Cu) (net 23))
 (segment (start 193.421 42.799) (end 186.69 49.53) (width 0.4) (layer B.Cu) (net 23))
 (segment (start 182.71316 53.34) (end 181.61 52.23684) (width 0.4) (layer B.Cu) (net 23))
 (segment (start 186.69 49.53) (end 186.69 52.07) (width 0.4) (layer B.Cu) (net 23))
 (segment (start 185.42 53.34) (end 182.71316 53.34) (width 0.4) (layer B.Cu) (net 23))
 (segment (start 181.61 52.23684) (end 181.61 50.8) (width 0.4) (layer B.Cu) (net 23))
 (segment (start 152.4 33.401) (end 156.591 33.401) (width 0.4) (layer B.Cu) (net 18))
 (segment (start 156.591 33.401) (end 173.99 50.8) (width 0.4) (layer B.Cu) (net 18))
 (segment (start 171.45 50.8) (end 163.449 42.799) (width 0.4) (layer B.Cu) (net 19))
 (segment (start 163.449 42.799) (end 152.4 42.799) (width 0.4) (layer B.Cu) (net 19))
 (segment (start 181.61 43.989398) (end 181.61 48.26) (width 0.4) (layer B.Cu) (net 20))
 (segment (start 181.61 48.26) (end 179.07 50.8) (width 0.4) (layer B.Cu) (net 20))
 (segment (start 174.009 40.64) (end 178.260602 40.64) (width 0.4) (layer B.Cu) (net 20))
 (segment (start 178.260602 40.64) (end 181.61 43.989398) (width 0.4) (layer B.Cu) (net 20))
 (segment (start 171.45 38.081) (end 174.009 40.64) (width 0.4) (layer B.Cu) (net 20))
 (segment (start 177.8 33.401) (end 176.13 33.401) (width 0.4) (layer B.Cu) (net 20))
 (segment (start 176.13 33.401) (end 171.45 38.081) (width 0.4) (layer B.Cu) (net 20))
 (segment (start 177.8 42.799) (end 177.8 49.53) (width 0.4) (layer B.Cu) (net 21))
 (segment (start 177.8 49.53) (end 176.53 50.8) (width 0.4) (layer B.Cu) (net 21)))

